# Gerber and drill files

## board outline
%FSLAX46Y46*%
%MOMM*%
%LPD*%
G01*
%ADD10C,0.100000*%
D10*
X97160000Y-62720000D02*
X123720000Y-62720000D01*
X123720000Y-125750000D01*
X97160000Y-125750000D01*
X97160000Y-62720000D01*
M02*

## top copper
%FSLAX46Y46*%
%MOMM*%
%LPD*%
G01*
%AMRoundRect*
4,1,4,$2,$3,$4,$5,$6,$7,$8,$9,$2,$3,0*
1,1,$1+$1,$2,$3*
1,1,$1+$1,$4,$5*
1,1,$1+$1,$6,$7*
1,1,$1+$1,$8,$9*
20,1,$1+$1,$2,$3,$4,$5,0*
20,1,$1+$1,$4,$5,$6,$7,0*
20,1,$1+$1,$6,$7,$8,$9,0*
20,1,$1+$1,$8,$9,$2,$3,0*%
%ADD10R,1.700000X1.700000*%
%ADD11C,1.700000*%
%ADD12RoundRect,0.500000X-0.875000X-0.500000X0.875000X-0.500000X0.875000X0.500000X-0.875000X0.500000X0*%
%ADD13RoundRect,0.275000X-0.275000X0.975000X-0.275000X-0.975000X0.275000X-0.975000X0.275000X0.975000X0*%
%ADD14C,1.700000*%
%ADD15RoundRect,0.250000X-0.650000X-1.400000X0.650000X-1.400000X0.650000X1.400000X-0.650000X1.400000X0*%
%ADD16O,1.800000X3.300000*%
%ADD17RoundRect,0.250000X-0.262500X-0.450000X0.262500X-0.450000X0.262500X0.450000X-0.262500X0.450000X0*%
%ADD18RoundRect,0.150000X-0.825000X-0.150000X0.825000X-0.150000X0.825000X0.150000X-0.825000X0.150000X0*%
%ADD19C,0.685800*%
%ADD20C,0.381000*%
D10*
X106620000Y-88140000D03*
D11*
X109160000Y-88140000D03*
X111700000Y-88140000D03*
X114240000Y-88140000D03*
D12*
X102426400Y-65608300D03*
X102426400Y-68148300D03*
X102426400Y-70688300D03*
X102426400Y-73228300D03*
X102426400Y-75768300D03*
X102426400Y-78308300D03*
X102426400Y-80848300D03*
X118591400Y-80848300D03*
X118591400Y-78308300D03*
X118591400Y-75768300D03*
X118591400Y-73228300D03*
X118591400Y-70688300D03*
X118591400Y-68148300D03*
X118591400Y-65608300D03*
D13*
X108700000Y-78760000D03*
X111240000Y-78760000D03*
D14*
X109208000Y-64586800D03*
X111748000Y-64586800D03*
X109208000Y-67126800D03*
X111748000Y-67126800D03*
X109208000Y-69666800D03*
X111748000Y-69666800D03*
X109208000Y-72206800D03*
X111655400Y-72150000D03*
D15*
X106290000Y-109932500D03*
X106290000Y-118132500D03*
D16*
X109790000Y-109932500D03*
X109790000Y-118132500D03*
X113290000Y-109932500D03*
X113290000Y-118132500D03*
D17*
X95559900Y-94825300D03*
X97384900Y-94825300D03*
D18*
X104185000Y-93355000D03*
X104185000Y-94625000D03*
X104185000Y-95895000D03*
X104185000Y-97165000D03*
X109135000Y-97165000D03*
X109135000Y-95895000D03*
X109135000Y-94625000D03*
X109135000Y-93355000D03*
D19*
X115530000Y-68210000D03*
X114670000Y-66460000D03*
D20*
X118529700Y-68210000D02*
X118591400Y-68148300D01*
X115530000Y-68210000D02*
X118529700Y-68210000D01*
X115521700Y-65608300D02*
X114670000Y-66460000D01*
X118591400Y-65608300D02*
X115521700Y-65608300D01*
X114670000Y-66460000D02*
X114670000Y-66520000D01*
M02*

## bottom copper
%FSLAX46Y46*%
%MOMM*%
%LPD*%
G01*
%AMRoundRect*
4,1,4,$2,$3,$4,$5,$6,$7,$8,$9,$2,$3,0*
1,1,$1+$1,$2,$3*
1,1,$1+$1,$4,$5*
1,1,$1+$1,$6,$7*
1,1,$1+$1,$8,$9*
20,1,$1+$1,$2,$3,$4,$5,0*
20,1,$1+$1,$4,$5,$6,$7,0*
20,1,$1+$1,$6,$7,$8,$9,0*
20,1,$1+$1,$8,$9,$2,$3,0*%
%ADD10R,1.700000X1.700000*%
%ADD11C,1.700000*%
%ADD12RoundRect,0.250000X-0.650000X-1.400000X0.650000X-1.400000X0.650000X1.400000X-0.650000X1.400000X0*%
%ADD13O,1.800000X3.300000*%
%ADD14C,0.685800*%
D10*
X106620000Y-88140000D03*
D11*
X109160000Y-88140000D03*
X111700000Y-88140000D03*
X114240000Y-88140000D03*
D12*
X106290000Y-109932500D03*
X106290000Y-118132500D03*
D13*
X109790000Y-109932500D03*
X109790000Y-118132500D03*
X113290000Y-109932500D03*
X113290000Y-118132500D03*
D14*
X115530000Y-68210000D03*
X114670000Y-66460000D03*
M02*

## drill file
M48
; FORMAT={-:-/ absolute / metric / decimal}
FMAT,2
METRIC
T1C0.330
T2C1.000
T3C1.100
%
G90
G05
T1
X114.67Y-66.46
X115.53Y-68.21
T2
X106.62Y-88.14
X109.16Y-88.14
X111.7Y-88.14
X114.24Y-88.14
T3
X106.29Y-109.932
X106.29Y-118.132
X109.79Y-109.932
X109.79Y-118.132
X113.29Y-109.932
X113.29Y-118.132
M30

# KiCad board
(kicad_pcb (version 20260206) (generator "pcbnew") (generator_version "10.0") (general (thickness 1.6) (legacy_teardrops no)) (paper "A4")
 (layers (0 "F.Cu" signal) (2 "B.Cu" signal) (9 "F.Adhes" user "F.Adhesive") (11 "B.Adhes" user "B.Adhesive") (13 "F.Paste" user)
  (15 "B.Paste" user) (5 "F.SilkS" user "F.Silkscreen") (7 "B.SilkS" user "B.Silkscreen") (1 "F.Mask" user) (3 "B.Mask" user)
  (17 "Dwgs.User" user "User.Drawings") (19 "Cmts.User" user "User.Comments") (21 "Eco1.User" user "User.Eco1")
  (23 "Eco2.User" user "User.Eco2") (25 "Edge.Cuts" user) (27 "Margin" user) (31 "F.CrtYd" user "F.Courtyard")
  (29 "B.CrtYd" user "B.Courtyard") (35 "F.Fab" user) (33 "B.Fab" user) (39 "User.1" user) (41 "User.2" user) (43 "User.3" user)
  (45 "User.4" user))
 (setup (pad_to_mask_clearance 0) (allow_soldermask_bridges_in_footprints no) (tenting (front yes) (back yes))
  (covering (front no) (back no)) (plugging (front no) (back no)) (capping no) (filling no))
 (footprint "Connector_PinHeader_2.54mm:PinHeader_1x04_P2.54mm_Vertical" (layer "F.Cu") (at 106.62 88.14 90)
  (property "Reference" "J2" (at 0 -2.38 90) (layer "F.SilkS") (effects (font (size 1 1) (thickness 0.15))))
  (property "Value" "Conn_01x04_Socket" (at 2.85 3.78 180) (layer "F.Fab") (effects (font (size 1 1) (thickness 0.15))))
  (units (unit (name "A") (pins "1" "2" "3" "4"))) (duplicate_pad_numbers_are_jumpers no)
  (pad "1" thru_hole rect (at 0 0 90) (size 1.7 1.7) (drill 1) (layers "*.Cu" "*.Mask") (remove_unused_layers no) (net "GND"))
  (pad "2" thru_hole circle (at 0 2.54 90) (size 1.7 1.7) (drill 1) (layers "*.Cu" "*.Mask") (remove_unused_layers no) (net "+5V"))
  (pad "3" thru_hole circle (at 0 5.08 90) (size 1.7 1.7) (drill 1) (layers "*.Cu" "*.Mask") (remove_unused_layers no) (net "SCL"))
  (pad "4" thru_hole circle (at 0 7.62 90) (size 1.7 1.7) (drill 1) (layers "*.Cu" "*.Mask") (remove_unused_layers no) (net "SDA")))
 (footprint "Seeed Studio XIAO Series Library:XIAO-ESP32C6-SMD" (layer "F.Cu") (at 110.708 73.2068)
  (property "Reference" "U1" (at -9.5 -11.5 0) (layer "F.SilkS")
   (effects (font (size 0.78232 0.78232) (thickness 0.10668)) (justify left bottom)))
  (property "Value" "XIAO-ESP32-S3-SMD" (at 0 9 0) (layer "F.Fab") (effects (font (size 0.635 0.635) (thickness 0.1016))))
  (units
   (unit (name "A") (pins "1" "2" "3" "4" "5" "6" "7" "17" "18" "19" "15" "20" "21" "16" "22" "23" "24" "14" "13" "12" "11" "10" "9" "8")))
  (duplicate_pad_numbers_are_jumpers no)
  (pad "1" smd roundrect (at -8.2816 -7.5985) (size 2.75 2) (layers "F.Cu" "F.Mask" "F.Paste") (roundrect_rratio 0.25)
   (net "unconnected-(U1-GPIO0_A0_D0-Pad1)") (solder_mask_margin 0.0508) (thermal_bridge_angle 45))
  (pad "2" smd roundrect (at -8.2816 -5.0585) (size 2.75 2) (layers "F.Cu" "F.Mask" "F.Paste") (roundrect_rratio 0.25)
   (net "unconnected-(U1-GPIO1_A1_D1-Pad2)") (solder_mask_margin 0.0508) (thermal_bridge_angle 45))
  (pad "3" smd roundrect (at -8.2816 -2.5185) (size 2.75 2) (layers "F.Cu" "F.Mask" "F.Paste") (roundrect_rratio 0.25) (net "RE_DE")
   (solder_mask_margin 0.0508) (thermal_bridge_angle 45))
  (pad "4" smd roundrect (at -8.2816 0.0215) (size 2.75 2) (layers "F.Cu" "F.Mask" "F.Paste") (roundrect_rratio 0.25)
   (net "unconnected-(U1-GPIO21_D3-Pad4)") (solder_mask_margin 0.0508) (thermal_bridge_angle 45))
  (pad "5" smd roundrect (at -8.2816 2.5615) (size 2.75 2) (layers "F.Cu" "F.Mask" "F.Paste") (roundrect_rratio 0.25) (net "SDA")
   (solder_mask_margin 0.0508) (thermal_bridge_angle 45))
  (pad "6" smd roundrect (at -8.2816 5.1015) (size 2.75 2) (layers "F.Cu" "F.Mask" "F.Paste") (roundrect_rratio 0.25) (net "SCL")
   (solder_mask_margin 0.0508) (thermal_bridge_angle 45))
  (pad "7" smd roundrect (at -8.2816 7.6415) (size 2.75 2) (layers "F.Cu" "F.Mask" "F.Paste") (roundrect_rratio 0.25) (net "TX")
   (solder_mask_margin 0.0508) (thermal_bridge_angle 45))
  (pad "8" smd roundrect (at 7.8834 7.6415) (size 2.75 2) (layers "F.Cu" "F.Mask" "F.Paste") (roundrect_rratio 0.25) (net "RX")
   (solder_mask_margin 0.0508) (thermal_bridge_angle 45))
  (pad "9" smd roundrect (at 7.8834 5.1015) (size 2.75 2) (layers "F.Cu" "F.Mask" "F.Paste") (roundrect_rratio 0.25)
   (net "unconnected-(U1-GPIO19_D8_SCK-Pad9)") (solder_mask_margin 0.0508) (thermal_bridge_angle 45))
  (pad "10" smd roundrect (at 7.8834 2.5615) (size 2.75 2) (layers "F.Cu" "F.Mask" "F.Paste") (roundrect_rratio 0.25)
   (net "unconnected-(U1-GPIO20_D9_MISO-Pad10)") (solder_mask_margin 0.0508) (thermal_bridge_angle 45))
  (pad "11" smd roundrect (at 7.8834 0.0215) (size 2.75 2) (layers "F.Cu" "F.Mask" "F.Paste") (roundrect_rratio 0.25)
   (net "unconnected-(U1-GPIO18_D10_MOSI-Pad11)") (solder_mask_margin 0.0508) (thermal_bridge_angle 45))
  (pad "12" smd roundrect (at 7.8834 -2.5185) (size 2.75 2) (layers "F.Cu" "F.Mask" "F.Paste") (roundrect_rratio 0.25)
   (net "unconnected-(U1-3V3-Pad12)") (solder_mask_margin 0.0508) (thermal_bridge_angle 45))
  (pad "13" smd roundrect (at 7.8834 -5.0585) (size 2.75 2) (layers "F.Cu" "F.Mask" "F.Paste") (roundrect_rratio 0.25) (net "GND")
   (solder_mask_margin 0.0508) (thermal_bridge_angle 45))
  (pad "14" smd roundrect (at 7.8834 -7.5985) (size 2.75 2) (layers "F.Cu" "F.Mask" "F.Paste") (roundrect_rratio 0.25) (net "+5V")
   (solder_mask_margin 0.0508) (thermal_bridge_angle 45))
  (pad "15" smd roundrect (at -2.008 5.5532 270) (size 2.5 1.1) (layers "F.Cu" "F.Mask" "F.Paste") (roundrect_rratio 0.25)
   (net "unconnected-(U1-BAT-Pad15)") (solder_mask_margin 0.0508) (thermal_bridge_angle 45))
  (pad "16" smd roundrect (at 0.532 5.5532 270) (size 2.5 1.1) (layers "F.Cu" "F.Mask" "F.Paste") (roundrect_rratio 0.25)
   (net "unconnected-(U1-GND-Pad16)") (solder_mask_margin 0.0508) (thermal_bridge_angle 45))
  (pad "17" smd circle (at -1.5 -8.62) (size 1.7 1.7) (layers "F.Cu" "F.Mask" "F.Paste") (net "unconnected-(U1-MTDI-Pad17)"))
  (pad "18" smd circle (at 1.04 -8.62) (size 1.7 1.7) (layers "F.Cu" "F.Mask" "F.Paste") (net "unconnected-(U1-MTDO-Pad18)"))
  (pad "19" smd circle (at -1.5 -6.08) (size 1.7 1.7) (layers "F.Cu" "F.Mask" "F.Paste") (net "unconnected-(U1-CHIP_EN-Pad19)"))
  (pad "20" smd circle (at 1.04 -6.08) (size 1.7 1.7) (layers "F.Cu" "F.Mask" "F.Paste") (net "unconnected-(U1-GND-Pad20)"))
  (pad "21" smd circle (at -1.5 -3.54) (size 1.7 1.7) (layers "F.Cu" "F.Mask" "F.Paste") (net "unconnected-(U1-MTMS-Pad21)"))
  (pad "22" smd circle (at 1.04 -3.54) (size 1.7 1.7) (layers "F.Cu" "F.Mask" "F.Paste") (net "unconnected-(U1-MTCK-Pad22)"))
  (pad "23" smd circle (at -1.5 -1) (size 1.7 1.7) (layers "F.Cu" "F.Mask" "F.Paste") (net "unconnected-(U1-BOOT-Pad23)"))
  (pad "24" smd circle (at 0.9474 -1.0568) (size 1.7 1.7) (layers "F.Cu" "F.Mask" "F.Paste") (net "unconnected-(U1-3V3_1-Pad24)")))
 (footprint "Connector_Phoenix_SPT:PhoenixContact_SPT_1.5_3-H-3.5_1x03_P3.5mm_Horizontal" (layer "F.Cu") (at 106.29 109.9325)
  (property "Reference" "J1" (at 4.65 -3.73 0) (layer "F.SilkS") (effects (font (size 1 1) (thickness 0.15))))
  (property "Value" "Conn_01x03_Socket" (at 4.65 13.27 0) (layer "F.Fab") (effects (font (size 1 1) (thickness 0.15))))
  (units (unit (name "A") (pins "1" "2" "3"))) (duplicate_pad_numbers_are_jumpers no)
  (pad "1" thru_hole roundrect (at 0 0) (size 1.8 3.3) (drill 1.1) (layers "*.Cu" "*.Mask") (remove_unused_layers no)
   (roundrect_rratio 0.138889) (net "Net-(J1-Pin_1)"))
  (pad "1" thru_hole roundrect (at 0 8.2) (size 1.8 3.3) (drill 1.1) (layers "*.Cu" "*.Mask") (remove_unused_layers no)
   (roundrect_rratio 0.138889) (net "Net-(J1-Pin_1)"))
  (pad "2" thru_hole oval (at 3.5 0) (size 1.8 3.3) (drill 1.1) (layers "*.Cu" "*.Mask") (remove_unused_layers no) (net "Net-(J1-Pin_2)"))
  (pad "2" thru_hole oval (at 3.5 8.2) (size 1.8 3.3) (drill 1.1) (layers "*.Cu" "*.Mask") (remove_unused_layers no) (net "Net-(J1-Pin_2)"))
  (pad "3" thru_hole oval (at 7 0) (size 1.8 3.3) (drill 1.1) (layers "*.Cu" "*.Mask") (remove_unused_layers no) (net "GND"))
  (pad "3" thru_hole oval (at 7 8.2) (size 1.8 3.3) (drill 1.1) (layers "*.Cu" "*.Mask") (remove_unused_layers no) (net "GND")))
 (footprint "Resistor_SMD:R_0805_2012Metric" (layer "F.Cu") (at 96.4724 94.8253)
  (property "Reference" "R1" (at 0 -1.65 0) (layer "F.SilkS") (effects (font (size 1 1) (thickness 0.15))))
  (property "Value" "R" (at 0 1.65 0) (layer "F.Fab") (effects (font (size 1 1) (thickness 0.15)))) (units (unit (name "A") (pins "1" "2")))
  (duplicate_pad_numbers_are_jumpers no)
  (pad "1" smd roundrect (at -0.9125 0) (size 1.025 1.4) (layers "F.Cu" "F.Mask" "F.Paste") (roundrect_rratio 0.243902)
   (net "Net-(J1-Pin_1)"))
  (pad "2" smd roundrect (at 0.9125 0) (size 1.025 1.4) (layers "F.Cu" "F.Mask" "F.Paste") (roundrect_rratio 0.243902)
   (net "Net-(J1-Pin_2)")))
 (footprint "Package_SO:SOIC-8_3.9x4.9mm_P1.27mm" (layer "F.Cu") (at 106.66 95.26)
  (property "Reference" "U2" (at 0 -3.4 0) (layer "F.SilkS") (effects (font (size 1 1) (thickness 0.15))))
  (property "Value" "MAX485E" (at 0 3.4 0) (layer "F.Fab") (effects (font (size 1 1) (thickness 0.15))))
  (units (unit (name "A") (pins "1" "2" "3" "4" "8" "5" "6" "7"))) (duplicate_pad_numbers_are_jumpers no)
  (pad "1" smd roundrect (at -2.475 -1.905) (size 1.95 0.6) (layers "F.Cu" "F.Mask" "F.Paste") (roundrect_rratio 0.25) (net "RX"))
  (pad "2" smd roundrect (at -2.475 -0.635) (size 1.95 0.6) (layers "F.Cu" "F.Mask" "F.Paste") (roundrect_rratio 0.25) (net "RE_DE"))
  (pad "3" smd roundrect (at -2.475 0.635) (size 1.95 0.6) (layers "F.Cu" "F.Mask" "F.Paste") (roundrect_rratio 0.25) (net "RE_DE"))
  (pad "4" smd roundrect (at -2.475 1.905) (size 1.95 0.6) (layers "F.Cu" "F.Mask" "F.Paste") (roundrect_rratio 0.25) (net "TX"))
  (pad "5" smd roundrect (at 2.475 1.905) (size 1.95 0.6) (layers "F.Cu" "F.Mask" "F.Paste") (roundrect_rratio 0.25) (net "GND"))
  (pad "6" smd roundrect (at 2.475 0.635) (size 1.95 0.6) (layers "F.Cu" "F.Mask" "F.Paste") (roundrect_rratio 0.25) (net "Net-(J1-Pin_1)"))
  (pad "7" smd roundrect (at 2.475 -0.635) (size 1.95 0.6) (layers "F.Cu" "F.Mask" "F.Paste") (roundrect_rratio 0.25) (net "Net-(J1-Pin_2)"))
  (pad "8" smd roundrect (at 2.475 -1.905) (size 1.95 0.6) (layers "F.Cu" "F.Mask" "F.Paste") (roundrect_rratio 0.25) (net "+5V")))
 (gr_rect (start 97.16 62.72) (end 123.72 125.75) (stroke (width 0.1) (type default)) (fill no) (layer "Edge.Cuts"))
 (segment (start 118.5297 68.21) (end 118.5914 68.1483) (width 0.381) (layer "F.Cu") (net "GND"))
 (segment (start 115.53 68.21) (end 118.5297 68.21) (width 0.381) (layer "F.Cu") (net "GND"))
 (via (at 115.53 68.21) (size 0.6858) (drill 0.3302) (layers "F.Cu" "B.Cu") (free yes) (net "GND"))
 (segment (start 115.5217 65.6083) (end 114.67 66.46) (width 0.381) (layer "F.Cu") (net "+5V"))
 (segment (start 118.5914 65.6083) (end 115.5217 65.6083) (width 0.381) (layer "F.Cu") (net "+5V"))
 (segment (start 114.67 66.46) (end 114.67 66.52) (width 0.381) (layer "F.Cu") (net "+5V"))
 (via (at 114.67 66.46) (size 0.6858) (drill 0.3302) (layers "F.Cu" "B.Cu") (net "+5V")))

